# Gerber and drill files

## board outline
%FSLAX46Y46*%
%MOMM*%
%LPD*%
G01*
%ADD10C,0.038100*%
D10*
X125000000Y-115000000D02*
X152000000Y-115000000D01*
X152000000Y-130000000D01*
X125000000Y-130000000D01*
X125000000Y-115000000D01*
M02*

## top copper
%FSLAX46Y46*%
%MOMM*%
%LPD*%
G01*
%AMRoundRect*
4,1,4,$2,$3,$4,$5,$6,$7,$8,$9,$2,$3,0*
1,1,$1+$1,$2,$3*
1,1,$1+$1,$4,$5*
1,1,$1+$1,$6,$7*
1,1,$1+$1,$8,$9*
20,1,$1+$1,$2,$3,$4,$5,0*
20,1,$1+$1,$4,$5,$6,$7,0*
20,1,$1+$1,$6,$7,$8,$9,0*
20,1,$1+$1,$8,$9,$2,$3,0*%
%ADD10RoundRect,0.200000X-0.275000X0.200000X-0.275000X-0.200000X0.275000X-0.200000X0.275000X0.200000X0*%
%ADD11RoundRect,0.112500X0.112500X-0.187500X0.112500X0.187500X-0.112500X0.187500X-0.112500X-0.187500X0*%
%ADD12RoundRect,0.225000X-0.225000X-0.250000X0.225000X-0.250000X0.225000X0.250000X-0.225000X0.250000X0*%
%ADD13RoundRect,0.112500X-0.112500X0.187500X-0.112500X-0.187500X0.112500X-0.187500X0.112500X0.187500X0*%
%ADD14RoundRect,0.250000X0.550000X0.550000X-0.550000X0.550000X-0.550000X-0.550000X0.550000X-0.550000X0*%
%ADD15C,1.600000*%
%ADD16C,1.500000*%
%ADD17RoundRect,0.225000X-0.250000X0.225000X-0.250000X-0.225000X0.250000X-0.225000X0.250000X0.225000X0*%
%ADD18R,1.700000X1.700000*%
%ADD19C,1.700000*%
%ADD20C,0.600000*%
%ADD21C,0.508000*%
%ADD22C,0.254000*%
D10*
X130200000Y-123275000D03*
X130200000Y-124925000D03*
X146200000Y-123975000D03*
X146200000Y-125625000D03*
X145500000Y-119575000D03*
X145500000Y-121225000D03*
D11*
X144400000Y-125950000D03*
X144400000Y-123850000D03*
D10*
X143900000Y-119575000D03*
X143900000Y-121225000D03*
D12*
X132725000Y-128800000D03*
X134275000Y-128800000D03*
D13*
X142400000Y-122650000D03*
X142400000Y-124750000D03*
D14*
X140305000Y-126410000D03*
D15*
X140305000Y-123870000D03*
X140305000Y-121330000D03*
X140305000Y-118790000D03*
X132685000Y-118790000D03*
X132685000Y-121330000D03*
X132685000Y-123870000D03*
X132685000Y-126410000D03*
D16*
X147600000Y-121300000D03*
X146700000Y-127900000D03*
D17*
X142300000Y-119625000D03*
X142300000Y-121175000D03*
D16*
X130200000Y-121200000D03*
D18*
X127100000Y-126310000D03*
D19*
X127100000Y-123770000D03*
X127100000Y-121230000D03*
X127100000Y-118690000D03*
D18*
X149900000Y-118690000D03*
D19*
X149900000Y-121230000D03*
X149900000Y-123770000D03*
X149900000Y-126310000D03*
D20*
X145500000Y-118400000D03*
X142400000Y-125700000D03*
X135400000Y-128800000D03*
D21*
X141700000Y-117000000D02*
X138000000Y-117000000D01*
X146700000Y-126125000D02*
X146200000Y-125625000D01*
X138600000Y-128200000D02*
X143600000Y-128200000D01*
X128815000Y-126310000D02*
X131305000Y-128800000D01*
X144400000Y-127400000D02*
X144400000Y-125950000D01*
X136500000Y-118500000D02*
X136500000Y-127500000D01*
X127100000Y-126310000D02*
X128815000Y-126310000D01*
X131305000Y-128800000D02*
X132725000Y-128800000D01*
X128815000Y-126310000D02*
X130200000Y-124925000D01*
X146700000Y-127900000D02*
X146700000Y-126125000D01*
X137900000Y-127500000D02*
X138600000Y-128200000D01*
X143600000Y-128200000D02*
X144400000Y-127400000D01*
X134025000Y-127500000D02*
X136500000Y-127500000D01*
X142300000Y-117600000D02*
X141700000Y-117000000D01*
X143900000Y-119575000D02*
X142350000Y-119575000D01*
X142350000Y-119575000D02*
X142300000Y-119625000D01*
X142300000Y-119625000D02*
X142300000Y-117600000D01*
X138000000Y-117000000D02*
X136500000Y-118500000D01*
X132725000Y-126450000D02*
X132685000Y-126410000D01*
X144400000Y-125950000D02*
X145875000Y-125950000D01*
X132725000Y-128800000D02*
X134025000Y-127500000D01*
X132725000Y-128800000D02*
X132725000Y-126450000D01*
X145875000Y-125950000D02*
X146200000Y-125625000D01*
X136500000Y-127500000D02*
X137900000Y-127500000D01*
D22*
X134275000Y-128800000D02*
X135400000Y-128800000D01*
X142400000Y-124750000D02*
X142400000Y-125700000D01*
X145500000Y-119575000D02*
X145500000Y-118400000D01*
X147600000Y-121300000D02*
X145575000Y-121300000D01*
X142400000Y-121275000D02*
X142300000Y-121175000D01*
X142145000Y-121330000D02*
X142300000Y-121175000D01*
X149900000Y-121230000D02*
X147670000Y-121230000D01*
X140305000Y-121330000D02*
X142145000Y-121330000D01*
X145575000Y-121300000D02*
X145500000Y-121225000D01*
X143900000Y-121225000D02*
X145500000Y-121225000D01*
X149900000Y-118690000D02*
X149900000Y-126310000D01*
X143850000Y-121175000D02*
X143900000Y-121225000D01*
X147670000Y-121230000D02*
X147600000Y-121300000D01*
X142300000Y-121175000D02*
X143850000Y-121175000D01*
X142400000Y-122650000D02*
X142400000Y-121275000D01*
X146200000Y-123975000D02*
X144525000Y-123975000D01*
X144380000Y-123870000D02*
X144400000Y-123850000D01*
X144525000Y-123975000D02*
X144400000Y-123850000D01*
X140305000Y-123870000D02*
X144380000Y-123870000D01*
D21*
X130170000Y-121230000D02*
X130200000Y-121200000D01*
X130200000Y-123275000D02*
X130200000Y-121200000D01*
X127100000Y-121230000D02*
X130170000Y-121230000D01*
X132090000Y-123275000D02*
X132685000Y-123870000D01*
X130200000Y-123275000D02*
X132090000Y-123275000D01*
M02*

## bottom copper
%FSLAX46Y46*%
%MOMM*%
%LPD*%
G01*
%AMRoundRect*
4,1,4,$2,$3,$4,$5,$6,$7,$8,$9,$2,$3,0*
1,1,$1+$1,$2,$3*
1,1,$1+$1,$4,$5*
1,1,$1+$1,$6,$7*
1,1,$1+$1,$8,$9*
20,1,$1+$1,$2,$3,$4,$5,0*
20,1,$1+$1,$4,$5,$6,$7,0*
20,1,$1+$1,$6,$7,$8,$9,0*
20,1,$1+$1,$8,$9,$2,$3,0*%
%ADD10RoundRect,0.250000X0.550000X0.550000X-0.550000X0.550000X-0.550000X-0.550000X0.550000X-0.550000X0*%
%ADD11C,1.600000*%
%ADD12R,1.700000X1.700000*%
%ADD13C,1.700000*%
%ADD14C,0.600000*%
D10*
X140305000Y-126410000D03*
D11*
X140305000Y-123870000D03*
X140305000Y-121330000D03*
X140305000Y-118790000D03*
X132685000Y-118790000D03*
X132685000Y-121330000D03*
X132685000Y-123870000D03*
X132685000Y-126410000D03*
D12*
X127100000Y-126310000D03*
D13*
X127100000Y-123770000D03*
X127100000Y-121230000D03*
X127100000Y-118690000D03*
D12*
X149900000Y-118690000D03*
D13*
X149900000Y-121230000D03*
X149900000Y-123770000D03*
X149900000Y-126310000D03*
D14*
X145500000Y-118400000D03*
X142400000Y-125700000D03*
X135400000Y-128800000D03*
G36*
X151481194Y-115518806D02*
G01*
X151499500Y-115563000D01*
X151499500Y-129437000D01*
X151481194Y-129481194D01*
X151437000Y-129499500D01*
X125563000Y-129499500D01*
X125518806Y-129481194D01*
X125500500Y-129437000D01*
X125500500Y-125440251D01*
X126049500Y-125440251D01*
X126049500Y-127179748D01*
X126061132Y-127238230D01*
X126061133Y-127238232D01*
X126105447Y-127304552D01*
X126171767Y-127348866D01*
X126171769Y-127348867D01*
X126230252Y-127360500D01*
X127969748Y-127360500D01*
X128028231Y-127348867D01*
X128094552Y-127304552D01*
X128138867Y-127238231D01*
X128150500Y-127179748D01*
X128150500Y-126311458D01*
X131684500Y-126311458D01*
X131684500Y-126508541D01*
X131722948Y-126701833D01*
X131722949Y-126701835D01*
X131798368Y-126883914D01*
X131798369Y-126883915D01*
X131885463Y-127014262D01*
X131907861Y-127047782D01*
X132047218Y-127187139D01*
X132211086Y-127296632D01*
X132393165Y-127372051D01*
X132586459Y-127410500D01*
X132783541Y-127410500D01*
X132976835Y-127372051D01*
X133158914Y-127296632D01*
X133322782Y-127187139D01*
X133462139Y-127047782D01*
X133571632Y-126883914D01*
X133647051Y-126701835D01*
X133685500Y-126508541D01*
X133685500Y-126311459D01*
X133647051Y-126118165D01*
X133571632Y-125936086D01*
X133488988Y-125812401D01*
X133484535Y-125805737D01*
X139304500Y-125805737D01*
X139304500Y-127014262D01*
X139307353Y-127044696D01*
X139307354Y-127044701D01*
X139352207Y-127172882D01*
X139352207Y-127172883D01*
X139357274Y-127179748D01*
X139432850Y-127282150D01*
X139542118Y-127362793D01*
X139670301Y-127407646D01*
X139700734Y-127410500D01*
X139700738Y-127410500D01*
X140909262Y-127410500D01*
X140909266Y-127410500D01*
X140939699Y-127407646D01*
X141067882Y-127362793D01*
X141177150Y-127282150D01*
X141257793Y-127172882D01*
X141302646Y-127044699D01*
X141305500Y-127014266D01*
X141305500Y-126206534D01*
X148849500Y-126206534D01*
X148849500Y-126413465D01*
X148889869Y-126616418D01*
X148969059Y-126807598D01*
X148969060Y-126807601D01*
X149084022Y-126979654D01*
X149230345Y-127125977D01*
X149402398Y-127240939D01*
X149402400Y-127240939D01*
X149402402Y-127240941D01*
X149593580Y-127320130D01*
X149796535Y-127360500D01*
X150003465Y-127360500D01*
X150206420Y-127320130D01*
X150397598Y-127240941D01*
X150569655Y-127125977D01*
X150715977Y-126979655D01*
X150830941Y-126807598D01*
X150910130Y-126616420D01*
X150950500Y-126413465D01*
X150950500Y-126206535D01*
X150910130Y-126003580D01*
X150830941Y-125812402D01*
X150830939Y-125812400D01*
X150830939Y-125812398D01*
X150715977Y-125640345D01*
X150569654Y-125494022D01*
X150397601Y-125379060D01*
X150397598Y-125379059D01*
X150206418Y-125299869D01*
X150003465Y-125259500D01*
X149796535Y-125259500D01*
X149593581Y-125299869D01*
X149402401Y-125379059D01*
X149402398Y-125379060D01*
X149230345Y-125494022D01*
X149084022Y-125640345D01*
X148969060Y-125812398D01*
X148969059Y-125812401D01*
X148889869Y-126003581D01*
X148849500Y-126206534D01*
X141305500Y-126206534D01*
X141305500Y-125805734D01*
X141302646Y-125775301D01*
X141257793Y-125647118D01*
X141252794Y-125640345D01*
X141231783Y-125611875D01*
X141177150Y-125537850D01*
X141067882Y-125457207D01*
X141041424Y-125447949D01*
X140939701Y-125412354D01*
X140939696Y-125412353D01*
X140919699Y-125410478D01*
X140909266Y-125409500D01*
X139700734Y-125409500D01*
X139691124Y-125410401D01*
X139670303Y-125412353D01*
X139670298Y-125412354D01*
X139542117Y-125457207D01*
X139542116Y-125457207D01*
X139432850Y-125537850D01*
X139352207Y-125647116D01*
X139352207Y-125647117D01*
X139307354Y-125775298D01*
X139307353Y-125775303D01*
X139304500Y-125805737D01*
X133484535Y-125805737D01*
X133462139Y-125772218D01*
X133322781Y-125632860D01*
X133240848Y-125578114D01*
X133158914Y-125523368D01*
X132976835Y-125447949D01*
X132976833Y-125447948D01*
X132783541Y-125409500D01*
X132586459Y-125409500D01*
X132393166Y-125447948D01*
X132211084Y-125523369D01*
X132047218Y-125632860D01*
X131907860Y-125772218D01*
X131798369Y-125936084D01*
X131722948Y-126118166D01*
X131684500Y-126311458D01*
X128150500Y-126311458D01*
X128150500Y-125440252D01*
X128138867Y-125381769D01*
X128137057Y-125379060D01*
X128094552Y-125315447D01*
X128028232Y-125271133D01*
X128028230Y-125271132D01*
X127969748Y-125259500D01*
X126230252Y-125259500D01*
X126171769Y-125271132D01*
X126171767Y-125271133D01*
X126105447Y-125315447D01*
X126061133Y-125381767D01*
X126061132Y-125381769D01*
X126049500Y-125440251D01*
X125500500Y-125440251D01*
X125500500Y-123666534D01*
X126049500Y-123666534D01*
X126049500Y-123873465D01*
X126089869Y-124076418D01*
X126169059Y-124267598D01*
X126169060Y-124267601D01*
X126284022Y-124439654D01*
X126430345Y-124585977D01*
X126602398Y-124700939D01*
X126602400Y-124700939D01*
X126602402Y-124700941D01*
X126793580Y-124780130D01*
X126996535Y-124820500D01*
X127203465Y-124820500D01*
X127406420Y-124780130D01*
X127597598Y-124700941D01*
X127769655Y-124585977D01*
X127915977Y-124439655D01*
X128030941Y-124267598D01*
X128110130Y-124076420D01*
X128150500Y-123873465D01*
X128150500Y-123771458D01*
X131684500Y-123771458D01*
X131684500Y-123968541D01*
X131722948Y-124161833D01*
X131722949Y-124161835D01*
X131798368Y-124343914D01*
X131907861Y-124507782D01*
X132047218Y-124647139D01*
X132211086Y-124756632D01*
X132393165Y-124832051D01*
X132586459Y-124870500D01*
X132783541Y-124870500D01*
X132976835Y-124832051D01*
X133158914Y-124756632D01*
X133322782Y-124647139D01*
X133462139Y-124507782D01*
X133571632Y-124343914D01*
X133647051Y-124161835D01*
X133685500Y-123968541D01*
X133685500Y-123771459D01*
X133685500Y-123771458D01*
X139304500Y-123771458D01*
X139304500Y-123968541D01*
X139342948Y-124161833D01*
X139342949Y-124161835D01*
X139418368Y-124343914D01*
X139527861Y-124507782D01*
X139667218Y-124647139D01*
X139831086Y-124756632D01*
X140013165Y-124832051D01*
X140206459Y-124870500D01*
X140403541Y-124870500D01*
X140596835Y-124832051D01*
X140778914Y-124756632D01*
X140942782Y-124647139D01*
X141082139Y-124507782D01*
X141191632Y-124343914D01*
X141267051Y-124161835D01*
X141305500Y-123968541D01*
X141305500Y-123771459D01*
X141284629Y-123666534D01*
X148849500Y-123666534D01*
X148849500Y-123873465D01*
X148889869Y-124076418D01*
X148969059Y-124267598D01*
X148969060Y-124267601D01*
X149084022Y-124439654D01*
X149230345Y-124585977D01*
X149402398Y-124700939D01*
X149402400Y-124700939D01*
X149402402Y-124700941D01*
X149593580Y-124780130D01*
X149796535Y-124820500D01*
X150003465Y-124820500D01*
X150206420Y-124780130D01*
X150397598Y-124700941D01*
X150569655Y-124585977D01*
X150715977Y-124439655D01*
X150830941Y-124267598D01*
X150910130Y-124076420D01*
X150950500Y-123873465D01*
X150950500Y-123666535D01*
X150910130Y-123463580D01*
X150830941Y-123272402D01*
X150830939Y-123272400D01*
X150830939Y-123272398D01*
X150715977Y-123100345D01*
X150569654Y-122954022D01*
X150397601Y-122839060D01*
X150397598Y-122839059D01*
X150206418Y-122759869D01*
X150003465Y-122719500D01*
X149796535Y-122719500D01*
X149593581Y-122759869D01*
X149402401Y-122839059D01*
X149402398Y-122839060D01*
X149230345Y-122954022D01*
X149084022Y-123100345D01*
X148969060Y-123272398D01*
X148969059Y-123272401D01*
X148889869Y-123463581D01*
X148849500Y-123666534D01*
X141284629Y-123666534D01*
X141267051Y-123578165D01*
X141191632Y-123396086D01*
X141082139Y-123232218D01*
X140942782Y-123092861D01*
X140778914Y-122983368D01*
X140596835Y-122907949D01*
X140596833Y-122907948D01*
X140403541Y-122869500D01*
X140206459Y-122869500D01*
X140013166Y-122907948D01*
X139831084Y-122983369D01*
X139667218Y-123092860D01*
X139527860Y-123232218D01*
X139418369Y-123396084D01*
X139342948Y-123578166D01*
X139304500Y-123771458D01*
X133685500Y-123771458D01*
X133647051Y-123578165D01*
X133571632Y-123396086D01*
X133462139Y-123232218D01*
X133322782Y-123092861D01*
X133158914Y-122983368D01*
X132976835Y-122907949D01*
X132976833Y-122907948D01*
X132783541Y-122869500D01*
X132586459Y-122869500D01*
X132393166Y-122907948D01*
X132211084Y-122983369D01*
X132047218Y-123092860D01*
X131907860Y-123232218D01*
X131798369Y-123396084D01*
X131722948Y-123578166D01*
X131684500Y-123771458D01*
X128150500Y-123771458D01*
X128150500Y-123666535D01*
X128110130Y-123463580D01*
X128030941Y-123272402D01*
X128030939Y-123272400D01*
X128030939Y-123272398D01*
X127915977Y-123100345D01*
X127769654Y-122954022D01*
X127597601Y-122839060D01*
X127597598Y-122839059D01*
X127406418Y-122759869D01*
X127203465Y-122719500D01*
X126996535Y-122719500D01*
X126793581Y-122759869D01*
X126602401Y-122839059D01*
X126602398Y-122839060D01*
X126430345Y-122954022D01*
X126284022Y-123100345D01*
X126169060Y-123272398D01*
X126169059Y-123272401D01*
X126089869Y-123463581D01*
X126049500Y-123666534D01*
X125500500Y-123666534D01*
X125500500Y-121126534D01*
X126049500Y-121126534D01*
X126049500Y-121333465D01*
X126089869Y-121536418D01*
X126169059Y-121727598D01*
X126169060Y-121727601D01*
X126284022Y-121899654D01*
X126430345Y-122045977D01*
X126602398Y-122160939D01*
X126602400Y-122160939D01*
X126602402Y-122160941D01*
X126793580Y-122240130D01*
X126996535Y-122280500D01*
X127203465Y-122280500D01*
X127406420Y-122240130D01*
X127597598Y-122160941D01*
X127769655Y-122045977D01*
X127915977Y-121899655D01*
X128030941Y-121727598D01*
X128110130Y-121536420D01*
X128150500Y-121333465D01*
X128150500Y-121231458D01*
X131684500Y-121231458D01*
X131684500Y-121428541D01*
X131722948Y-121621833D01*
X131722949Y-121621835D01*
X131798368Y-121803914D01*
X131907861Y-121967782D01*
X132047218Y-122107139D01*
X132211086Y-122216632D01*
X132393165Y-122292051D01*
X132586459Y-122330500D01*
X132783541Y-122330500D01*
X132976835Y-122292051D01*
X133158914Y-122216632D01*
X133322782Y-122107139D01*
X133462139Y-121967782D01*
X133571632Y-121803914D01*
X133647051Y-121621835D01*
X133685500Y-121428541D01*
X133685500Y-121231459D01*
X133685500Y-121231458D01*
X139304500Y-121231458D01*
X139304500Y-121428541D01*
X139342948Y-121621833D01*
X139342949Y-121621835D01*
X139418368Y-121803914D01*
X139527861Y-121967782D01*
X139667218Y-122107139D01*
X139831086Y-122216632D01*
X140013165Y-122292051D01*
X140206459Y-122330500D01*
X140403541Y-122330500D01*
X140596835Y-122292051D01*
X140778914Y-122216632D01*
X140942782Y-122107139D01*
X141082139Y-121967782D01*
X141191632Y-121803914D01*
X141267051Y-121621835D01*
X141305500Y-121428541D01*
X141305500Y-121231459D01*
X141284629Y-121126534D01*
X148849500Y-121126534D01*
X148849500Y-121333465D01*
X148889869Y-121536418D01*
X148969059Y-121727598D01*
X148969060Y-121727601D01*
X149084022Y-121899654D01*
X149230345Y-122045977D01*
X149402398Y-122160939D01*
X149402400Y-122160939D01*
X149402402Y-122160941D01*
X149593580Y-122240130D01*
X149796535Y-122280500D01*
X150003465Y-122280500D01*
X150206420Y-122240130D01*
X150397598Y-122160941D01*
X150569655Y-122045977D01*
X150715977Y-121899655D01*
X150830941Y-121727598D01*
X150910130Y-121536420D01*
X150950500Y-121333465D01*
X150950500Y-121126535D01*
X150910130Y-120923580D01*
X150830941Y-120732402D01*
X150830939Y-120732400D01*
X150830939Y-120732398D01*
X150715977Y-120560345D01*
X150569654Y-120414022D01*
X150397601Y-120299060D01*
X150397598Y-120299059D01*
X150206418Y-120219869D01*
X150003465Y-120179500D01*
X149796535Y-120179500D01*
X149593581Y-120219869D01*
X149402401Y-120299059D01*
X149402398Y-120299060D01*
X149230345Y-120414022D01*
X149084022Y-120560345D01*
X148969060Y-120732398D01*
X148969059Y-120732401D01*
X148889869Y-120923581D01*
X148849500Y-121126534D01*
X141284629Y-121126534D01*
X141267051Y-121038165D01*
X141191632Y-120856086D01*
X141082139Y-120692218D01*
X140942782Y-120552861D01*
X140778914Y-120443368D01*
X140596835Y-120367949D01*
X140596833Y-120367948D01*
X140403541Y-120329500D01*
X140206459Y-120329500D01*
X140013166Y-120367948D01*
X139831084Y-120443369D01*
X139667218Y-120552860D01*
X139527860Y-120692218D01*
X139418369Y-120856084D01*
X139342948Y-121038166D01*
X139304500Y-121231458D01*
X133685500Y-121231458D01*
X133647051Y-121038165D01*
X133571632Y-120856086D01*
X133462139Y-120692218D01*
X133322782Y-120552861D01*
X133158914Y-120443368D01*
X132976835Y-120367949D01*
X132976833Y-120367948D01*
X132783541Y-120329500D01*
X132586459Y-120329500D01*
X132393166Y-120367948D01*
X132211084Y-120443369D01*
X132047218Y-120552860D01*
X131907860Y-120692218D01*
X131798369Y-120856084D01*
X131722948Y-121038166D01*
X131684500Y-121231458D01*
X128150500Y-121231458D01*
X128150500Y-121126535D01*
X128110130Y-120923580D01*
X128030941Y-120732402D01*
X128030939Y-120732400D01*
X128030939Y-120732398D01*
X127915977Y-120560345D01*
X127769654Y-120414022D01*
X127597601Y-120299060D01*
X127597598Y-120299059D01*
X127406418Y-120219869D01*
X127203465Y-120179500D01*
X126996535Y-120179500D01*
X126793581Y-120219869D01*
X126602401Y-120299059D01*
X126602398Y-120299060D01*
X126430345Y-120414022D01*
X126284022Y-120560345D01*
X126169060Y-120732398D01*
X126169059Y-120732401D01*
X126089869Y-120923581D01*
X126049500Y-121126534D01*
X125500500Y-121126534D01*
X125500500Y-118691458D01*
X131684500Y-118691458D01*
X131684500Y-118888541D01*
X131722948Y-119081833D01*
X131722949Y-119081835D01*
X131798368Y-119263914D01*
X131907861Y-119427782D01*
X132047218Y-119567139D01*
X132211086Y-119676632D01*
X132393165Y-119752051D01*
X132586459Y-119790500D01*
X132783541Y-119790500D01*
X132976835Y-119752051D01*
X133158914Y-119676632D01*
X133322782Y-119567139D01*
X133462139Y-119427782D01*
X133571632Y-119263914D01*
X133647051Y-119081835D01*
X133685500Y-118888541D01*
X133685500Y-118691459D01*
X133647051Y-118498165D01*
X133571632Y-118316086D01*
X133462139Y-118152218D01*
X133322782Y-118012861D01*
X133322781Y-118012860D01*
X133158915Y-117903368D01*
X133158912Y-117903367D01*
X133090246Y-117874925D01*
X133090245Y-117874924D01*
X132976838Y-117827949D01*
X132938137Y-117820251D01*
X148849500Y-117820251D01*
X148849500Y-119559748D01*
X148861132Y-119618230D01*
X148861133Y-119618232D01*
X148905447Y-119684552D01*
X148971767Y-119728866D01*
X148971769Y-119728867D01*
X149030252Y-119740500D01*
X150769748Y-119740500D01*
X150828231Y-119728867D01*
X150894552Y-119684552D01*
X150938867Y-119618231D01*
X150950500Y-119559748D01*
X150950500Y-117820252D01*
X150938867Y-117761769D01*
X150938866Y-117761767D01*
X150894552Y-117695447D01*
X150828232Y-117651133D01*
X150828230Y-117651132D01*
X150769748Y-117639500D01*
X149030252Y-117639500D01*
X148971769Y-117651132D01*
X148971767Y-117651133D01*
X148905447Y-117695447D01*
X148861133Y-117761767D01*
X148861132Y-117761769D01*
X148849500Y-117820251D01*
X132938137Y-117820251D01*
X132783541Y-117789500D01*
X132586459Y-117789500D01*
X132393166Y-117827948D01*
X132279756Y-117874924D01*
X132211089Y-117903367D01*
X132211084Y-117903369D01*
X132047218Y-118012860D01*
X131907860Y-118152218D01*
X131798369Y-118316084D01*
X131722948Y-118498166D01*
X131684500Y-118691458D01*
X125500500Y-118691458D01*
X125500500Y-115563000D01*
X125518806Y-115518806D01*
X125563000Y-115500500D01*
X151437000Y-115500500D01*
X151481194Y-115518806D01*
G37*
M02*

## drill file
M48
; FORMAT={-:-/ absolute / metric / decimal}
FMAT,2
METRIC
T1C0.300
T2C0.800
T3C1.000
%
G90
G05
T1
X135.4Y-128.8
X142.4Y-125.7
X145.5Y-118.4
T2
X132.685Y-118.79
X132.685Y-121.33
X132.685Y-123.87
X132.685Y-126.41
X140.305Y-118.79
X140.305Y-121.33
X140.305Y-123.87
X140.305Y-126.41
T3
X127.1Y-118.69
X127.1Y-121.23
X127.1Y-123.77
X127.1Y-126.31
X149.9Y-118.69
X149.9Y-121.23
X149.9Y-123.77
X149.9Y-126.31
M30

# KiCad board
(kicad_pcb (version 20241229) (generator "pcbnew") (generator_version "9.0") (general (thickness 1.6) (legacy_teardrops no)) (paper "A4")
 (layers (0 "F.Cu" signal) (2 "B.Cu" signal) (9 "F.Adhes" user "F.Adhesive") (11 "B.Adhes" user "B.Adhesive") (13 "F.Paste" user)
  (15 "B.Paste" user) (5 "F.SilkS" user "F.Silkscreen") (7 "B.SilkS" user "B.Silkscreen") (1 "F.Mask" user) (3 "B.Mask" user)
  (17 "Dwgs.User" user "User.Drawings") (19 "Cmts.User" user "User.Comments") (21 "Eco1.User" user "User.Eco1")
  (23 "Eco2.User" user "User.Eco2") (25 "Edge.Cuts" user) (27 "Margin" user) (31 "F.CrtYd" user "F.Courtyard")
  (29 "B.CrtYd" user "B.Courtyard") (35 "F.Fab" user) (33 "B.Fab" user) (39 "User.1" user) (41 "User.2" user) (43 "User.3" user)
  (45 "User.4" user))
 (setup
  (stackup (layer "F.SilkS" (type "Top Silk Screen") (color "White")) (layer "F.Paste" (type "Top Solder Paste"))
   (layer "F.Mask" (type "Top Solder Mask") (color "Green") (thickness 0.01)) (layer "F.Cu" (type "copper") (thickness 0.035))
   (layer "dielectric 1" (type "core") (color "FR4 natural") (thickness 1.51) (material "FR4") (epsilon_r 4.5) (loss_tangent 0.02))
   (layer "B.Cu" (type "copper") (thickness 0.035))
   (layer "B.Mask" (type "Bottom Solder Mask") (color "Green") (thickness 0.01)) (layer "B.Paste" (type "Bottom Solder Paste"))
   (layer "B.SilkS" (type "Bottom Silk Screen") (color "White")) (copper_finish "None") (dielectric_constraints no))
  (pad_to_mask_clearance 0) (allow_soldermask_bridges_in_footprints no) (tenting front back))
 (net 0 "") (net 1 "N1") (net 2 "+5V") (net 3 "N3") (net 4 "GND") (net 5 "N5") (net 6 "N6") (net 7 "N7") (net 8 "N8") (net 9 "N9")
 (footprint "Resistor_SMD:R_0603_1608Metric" (layer "F.Cu") (at 130.2 124.1 -90)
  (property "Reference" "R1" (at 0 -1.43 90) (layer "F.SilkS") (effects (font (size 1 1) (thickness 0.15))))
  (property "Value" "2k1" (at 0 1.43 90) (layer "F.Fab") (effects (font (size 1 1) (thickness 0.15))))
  (pad "1" smd roundrect (at -0.825 0 270) (size 0.8 0.95) (layers "F.Cu" "F.Mask" "F.Paste") (roundrect_rratio 0.25) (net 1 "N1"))
  (pad "2" smd roundrect (at 0.825 0 270) (size 0.8 0.95) (layers "F.Cu" "F.Mask" "F.Paste") (roundrect_rratio 0.25) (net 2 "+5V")))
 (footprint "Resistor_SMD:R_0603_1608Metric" (layer "F.Cu") (at 146.2 124.8 -90)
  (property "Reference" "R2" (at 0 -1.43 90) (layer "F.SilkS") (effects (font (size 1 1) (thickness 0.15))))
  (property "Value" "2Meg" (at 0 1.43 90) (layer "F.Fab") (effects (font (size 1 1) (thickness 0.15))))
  (pad "1" smd roundrect (at -0.825 0 270) (size 0.8 0.95) (layers "F.Cu" "F.Mask" "F.Paste") (roundrect_rratio 0.25) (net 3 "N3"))
  (pad "2" smd roundrect (at 0.825 0 270) (size 0.8 0.95) (layers "F.Cu" "F.Mask" "F.Paste") (roundrect_rratio 0.25) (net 2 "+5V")))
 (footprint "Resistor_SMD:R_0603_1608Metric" (layer "F.Cu") (at 145.5 120.4 -90)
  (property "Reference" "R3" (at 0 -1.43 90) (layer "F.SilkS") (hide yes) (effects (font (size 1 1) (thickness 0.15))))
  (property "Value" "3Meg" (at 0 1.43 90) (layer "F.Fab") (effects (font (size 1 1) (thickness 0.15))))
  (pad "1" smd roundrect (at -0.825 0 270) (size 0.8 0.95) (layers "F.Cu" "F.Mask" "F.Paste") (roundrect_rratio 0.25) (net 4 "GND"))
  (pad "2" smd roundrect (at 0.825 0 270) (size 0.8 0.95) (layers "F.Cu" "F.Mask" "F.Paste") (roundrect_rratio 0.25) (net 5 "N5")))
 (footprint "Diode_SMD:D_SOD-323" (layer "F.Cu") (at 144.4 124.9 90)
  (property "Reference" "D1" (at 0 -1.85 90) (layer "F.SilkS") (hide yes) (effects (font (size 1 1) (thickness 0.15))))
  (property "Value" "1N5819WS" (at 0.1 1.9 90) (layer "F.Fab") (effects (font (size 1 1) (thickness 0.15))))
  (pad "1" smd roundrect (at -1.05 0 90) (size 0.6 0.45) (layers "F.Cu" "F.Mask" "F.Paste") (roundrect_rratio 0.25) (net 2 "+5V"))
  (pad "2" smd roundrect (at 1.05 0 90) (size 0.6 0.45) (layers "F.Cu" "F.Mask" "F.Paste") (roundrect_rratio 0.25) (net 3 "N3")))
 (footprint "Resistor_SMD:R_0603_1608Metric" (layer "F.Cu") (at 143.9 120.4 -90)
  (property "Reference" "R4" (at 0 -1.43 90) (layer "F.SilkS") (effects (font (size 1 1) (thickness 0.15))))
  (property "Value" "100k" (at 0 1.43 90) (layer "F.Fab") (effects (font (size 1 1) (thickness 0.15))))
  (pad "1" smd roundrect (at -0.825 0 270) (size 0.8 0.95) (layers "F.Cu" "F.Mask" "F.Paste") (roundrect_rratio 0.25) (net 2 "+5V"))
  (pad "2" smd roundrect (at 0.825 0 270) (size 0.8 0.95) (layers "F.Cu" "F.Mask" "F.Paste") (roundrect_rratio 0.25) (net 5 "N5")))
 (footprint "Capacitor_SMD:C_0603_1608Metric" (layer "F.Cu") (at 133.5 128.8)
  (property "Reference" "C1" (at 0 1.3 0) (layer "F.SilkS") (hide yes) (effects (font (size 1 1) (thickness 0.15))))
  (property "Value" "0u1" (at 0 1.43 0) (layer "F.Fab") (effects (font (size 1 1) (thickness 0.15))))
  (pad "1" smd roundrect (at -0.775 0) (size 0.9 0.95) (layers "F.Cu" "F.Mask" "F.Paste") (roundrect_rratio 0.25) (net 2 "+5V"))
  (pad "2" smd roundrect (at 0.775 0) (size 0.9 0.95) (layers "F.Cu" "F.Mask" "F.Paste") (roundrect_rratio 0.25) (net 4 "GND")))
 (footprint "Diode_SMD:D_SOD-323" (layer "F.Cu") (at 142.4 123.7 -90)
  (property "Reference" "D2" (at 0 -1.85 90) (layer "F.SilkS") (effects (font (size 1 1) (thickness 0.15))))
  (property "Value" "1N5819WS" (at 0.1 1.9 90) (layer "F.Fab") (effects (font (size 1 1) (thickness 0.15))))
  (pad "1" smd roundrect (at -1.05 0 270) (size 0.6 0.45) (layers "F.Cu" "F.Mask" "F.Paste") (roundrect_rratio 0.25) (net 5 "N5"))
  (pad "2" smd roundrect (at 1.05 0 270) (size 0.6 0.45) (layers "F.Cu" "F.Mask" "F.Paste") (roundrect_rratio 0.25) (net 4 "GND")))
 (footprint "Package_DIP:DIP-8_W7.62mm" (layer "F.Cu") (at 140.305 126.41 180)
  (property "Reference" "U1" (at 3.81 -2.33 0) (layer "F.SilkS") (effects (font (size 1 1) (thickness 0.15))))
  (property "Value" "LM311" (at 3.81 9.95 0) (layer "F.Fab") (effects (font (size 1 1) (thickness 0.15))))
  (pad "1" thru_hole roundrect (at 0 0 180) (size 1.6 1.6) (drill 0.8) (layers "*.Cu" "*.Mask") (remove_unused_layers no)
   (roundrect_rratio 0.15625) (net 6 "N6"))
  (pad "2" thru_hole circle (at 0 2.54 180) (size 1.6 1.6) (drill 0.8) (layers "*.Cu" "*.Mask") (remove_unused_layers no) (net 3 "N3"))
  (pad "3" thru_hole circle (at 0 5.08 180) (size 1.6 1.6) (drill 0.8) (layers "*.Cu" "*.Mask") (remove_unused_layers no) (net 5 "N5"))
  (pad "4" thru_hole circle (at 0 7.62 180) (size 1.6 1.6) (drill 0.8) (layers "*.Cu" "*.Mask") (remove_unused_layers no) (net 4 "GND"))
  (pad "5" thru_hole circle (at 7.62 7.62 180) (size 1.6 1.6) (drill 0.8) (layers "*.Cu" "*.Mask") (remove_unused_layers no) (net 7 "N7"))
  (pad "6" thru_hole circle (at 7.62 5.08 180) (size 1.6 1.6) (drill 0.8) (layers "*.Cu" "*.Mask") (remove_unused_layers no) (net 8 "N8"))
  (pad "7" thru_hole circle (at 7.62 2.54 180) (size 1.6 1.6) (drill 0.8) (layers "*.Cu" "*.Mask") (remove_unused_layers no) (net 1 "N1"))
  (pad "8" thru_hole circle (at 7.62 0 180) (size 1.6 1.6) (drill 0.8) (layers "*.Cu" "*.Mask") (remove_unused_layers no) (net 2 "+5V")))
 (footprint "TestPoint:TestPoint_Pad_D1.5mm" (layer "F.Cu") (at 147.6 121.3)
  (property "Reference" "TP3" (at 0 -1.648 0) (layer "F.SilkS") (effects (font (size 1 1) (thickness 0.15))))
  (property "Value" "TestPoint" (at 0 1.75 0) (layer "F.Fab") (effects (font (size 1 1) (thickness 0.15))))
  (pad "1" smd circle (at 0 0) (size 1.5 1.5) (layers "F.Cu" "F.Mask") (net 5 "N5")))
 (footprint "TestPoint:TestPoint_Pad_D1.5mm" (layer "F.Cu") (at 146.7 127.9)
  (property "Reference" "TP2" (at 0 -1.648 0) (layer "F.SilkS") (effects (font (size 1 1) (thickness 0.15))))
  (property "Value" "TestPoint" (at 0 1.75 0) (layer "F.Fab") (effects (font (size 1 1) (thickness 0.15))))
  (pad "1" smd circle (at 0 0) (size 1.5 1.5) (layers "F.Cu" "F.Mask") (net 2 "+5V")))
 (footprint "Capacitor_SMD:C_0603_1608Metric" (layer "F.Cu") (at 142.3 120.4 -90)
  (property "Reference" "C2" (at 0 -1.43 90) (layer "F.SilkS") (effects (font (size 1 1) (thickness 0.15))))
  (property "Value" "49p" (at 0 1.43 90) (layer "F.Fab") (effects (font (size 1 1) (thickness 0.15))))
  (pad "1" smd roundrect (at -0.775 0 270) (size 0.9 0.95) (layers "F.Cu" "F.Mask" "F.Paste") (roundrect_rratio 0.25) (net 2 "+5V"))
  (pad "2" smd roundrect (at 0.775 0 270) (size 0.9 0.95) (layers "F.Cu" "F.Mask" "F.Paste") (roundrect_rratio 0.25) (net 5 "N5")))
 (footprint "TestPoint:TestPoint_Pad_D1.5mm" (layer "F.Cu") (at 130.2 121.2)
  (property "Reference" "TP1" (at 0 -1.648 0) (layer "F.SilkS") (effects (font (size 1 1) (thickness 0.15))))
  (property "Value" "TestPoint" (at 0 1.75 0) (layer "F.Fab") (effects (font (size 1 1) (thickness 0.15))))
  (pad "1" smd circle (at 0 0) (size 1.5 1.5) (layers "F.Cu" "F.Mask") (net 1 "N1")))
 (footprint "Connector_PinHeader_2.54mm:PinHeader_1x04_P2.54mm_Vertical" (layer "B.Cu") (at 127.1 126.31)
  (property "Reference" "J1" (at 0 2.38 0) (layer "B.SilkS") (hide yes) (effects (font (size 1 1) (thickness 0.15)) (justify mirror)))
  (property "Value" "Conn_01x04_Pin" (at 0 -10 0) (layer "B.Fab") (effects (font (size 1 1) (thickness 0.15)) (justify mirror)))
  (pad "1" thru_hole rect (at 0 0) (size 1.7 1.7) (drill 1) (layers "*.Cu" "*.Mask") (remove_unused_layers no) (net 2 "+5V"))
  (pad "2" thru_hole circle (at 0 -2.54) (size 1.7 1.7) (drill 1) (layers "*.Cu" "*.Mask") (remove_unused_layers no) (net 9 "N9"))
  (pad "3" thru_hole circle (at 0 -5.08) (size 1.7 1.7) (drill 1) (layers "*.Cu" "*.Mask") (remove_unused_layers no) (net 1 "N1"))
  (pad "4" thru_hole circle (at 0 -7.62) (size 1.7 1.7) (drill 1) (layers "*.Cu" "*.Mask") (remove_unused_layers no) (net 4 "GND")))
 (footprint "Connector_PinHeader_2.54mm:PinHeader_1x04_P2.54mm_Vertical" (layer "B.Cu") (at 149.9 118.69 180)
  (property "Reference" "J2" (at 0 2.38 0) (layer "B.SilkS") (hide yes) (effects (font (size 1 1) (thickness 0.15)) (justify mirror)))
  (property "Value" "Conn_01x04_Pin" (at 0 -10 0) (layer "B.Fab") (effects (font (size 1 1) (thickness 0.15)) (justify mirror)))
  (pad "1" thru_hole rect (at 0 0 180) (size 1.7 1.7) (drill 1) (layers "*.Cu" "*.Mask") (remove_unused_layers no) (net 5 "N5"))
  (pad "2" thru_hole circle (at 0 -2.54 180) (size 1.7 1.7) (drill 1) (layers "*.Cu" "*.Mask") (remove_unused_layers no) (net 5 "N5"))
  (pad "3" thru_hole circle (at 0 -5.08 180) (size 1.7 1.7) (drill 1) (layers "*.Cu" "*.Mask") (remove_unused_layers no) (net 5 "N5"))
  (pad "4" thru_hole circle (at 0 -7.62 180) (size 1.7 1.7) (drill 1) (layers "*.Cu" "*.Mask") (remove_unused_layers no) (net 5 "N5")))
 (gr_rect (start 125 115) (end 152 130) (stroke (width 0.0381) (type default)) (fill no) (layer "Edge.Cuts"))
 (segment (start 141.7 117) (end 138 117) (width 0.508) (layer "F.Cu") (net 2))
 (segment (start 146.7 126.125) (end 146.2 125.625) (width 0.508) (layer "F.Cu") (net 2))
 (segment (start 138.6 128.2) (end 143.6 128.2) (width 0.508) (layer "F.Cu") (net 2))
 (segment (start 128.815 126.31) (end 131.305 128.8) (width 0.508) (layer "F.Cu") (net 2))
 (segment (start 144.4 127.4) (end 144.4 125.95) (width 0.508) (layer "F.Cu") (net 2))
 (segment (start 136.5 118.5) (end 136.5 127.5) (width 0.508) (layer "F.Cu") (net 2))
 (segment (start 127.1 126.31) (end 128.815 126.31) (width 0.508) (layer "F.Cu") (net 2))
 (segment (start 131.305 128.8) (end 132.725 128.8) (width 0.508) (layer "F.Cu") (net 2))
 (segment (start 128.815 126.31) (end 130.2 124.925) (width 0.508) (layer "F.Cu") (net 2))
 (segment (start 146.7 127.9) (end 146.7 126.125) (width 0.508) (layer "F.Cu") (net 2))
 (segment (start 137.9 127.5) (end 138.6 128.2) (width 0.508) (layer "F.Cu") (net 2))
 (segment (start 143.6 128.2) (end 144.4 127.4) (width 0.508) (layer "F.Cu") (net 2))
 (segment (start 134.025 127.5) (end 136.5 127.5) (width 0.508) (layer "F.Cu") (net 2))
 (segment (start 142.3 117.6) (end 141.7 117) (width 0.508) (layer "F.Cu") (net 2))
 (segment (start 143.9 119.575) (end 142.35 119.575) (width 0.508) (layer "F.Cu") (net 2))
 (segment (start 142.35 119.575) (end 142.3 119.625) (width 0.508) (layer "F.Cu") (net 2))
 (segment (start 142.3 119.625) (end 142.3 117.6) (width 0.508) (layer "F.Cu") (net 2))
 (segment (start 138 117) (end 136.5 118.5) (width 0.508) (layer "F.Cu") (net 2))
 (segment (start 132.725 126.45) (end 132.685 126.41) (width 0.508) (layer "F.Cu") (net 2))
 (segment (start 144.4 125.95) (end 145.875 125.95) (width 0.508) (layer "F.Cu") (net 2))
 (segment (start 132.725 128.8) (end 134.025 127.5) (width 0.508) (layer "F.Cu") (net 2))
 (segment (start 132.725 128.8) (end 132.725 126.45) (width 0.508) (layer "F.Cu") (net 2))
 (segment (start 145.875 125.95) (end 146.2 125.625) (width 0.508) (layer "F.Cu") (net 2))
 (segment (start 136.5 127.5) (end 137.9 127.5) (width 0.508) (layer "F.Cu") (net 2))
 (segment (start 134.275 128.8) (end 135.4 128.8) (width 0.254) (layer "F.Cu") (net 4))
 (segment (start 142.4 124.75) (end 142.4 125.7) (width 0.254) (layer "F.Cu") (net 4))
 (segment (start 145.5 119.575) (end 145.5 118.4) (width 0.254) (layer "F.Cu") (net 4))
 (via (at 145.5 118.4) (size 0.6) (drill 0.3) (layers "F.Cu" "B.Cu") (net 4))
 (via (at 142.4 125.7) (size 0.6) (drill 0.3) (layers "F.Cu" "B.Cu") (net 4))
 (via (at 135.4 128.8) (size 0.6) (drill 0.3) (layers "F.Cu" "B.Cu") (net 4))
 (segment (start 147.6 121.3) (end 145.575 121.3) (width 0.254) (layer "F.Cu") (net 5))
 (segment (start 142.4 121.275) (end 142.3 121.175) (width 0.254) (layer "F.Cu") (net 5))
 (segment (start 142.145 121.33) (end 142.3 121.175) (width 0.254) (layer "F.Cu") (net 5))
 (segment (start 149.9 121.23) (end 147.67 121.23) (width 0.254) (layer "F.Cu") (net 5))
 (segment (start 140.305 121.33) (end 142.145 121.33) (width 0.254) (layer "F.Cu") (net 5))
 (segment (start 145.575 121.3) (end 145.5 121.225) (width 0.254) (layer "F.Cu") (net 5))
 (segment (start 143.9 121.225) (end 145.5 121.225) (width 0.254) (layer "F.Cu") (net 5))
 (segment (start 149.9 118.69) (end 149.9 126.31) (width 0.254) (layer "F.Cu") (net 5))
 (segment (start 143.85 121.175) (end 143.9 121.225) (width 0.254) (layer "F.Cu") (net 5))
 (segment (start 147.67 121.23) (end 147.6 121.3) (width 0.254) (layer "F.Cu") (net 5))
 (segment (start 142.3 121.175) (end 143.85 121.175) (width 0.254) (layer "F.Cu") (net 5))
 (segment (start 142.4 122.65) (end 142.4 121.275) (width 0.254) (layer "F.Cu") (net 5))
 (segment (start 146.2 123.975) (end 144.525 123.975) (width 0.254) (layer "F.Cu") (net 3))
 (segment (start 144.38 123.87) (end 144.4 123.85) (width 0.254) (layer "F.Cu") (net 3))
 (segment (start 144.525 123.975) (end 144.4 123.85) (width 0.254) (layer "F.Cu") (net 3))
 (segment (start 140.305 123.87) (end 144.38 123.87) (width 0.254) (layer "F.Cu") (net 3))
 (segment (start 130.17 121.23) (end 130.2 121.2) (width 0.508) (layer "F.Cu") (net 1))
 (segment (start 130.2 123.275) (end 130.2 121.2) (width 0.508) (layer "F.Cu") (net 1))
 (segment (start 127.1 121.23) (end 130.17 121.23) (width 0.508) (layer "F.Cu") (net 1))
 (segment (start 132.09 123.275) (end 132.685 123.87) (width 0.508) (layer "F.Cu") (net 1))
 (segment (start 130.2 123.275) (end 132.09 123.275) (width 0.508) (layer "F.Cu") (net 1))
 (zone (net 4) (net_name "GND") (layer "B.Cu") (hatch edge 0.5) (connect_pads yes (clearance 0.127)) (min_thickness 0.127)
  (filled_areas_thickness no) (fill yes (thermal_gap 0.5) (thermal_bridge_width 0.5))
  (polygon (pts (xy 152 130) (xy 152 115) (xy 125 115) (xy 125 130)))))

